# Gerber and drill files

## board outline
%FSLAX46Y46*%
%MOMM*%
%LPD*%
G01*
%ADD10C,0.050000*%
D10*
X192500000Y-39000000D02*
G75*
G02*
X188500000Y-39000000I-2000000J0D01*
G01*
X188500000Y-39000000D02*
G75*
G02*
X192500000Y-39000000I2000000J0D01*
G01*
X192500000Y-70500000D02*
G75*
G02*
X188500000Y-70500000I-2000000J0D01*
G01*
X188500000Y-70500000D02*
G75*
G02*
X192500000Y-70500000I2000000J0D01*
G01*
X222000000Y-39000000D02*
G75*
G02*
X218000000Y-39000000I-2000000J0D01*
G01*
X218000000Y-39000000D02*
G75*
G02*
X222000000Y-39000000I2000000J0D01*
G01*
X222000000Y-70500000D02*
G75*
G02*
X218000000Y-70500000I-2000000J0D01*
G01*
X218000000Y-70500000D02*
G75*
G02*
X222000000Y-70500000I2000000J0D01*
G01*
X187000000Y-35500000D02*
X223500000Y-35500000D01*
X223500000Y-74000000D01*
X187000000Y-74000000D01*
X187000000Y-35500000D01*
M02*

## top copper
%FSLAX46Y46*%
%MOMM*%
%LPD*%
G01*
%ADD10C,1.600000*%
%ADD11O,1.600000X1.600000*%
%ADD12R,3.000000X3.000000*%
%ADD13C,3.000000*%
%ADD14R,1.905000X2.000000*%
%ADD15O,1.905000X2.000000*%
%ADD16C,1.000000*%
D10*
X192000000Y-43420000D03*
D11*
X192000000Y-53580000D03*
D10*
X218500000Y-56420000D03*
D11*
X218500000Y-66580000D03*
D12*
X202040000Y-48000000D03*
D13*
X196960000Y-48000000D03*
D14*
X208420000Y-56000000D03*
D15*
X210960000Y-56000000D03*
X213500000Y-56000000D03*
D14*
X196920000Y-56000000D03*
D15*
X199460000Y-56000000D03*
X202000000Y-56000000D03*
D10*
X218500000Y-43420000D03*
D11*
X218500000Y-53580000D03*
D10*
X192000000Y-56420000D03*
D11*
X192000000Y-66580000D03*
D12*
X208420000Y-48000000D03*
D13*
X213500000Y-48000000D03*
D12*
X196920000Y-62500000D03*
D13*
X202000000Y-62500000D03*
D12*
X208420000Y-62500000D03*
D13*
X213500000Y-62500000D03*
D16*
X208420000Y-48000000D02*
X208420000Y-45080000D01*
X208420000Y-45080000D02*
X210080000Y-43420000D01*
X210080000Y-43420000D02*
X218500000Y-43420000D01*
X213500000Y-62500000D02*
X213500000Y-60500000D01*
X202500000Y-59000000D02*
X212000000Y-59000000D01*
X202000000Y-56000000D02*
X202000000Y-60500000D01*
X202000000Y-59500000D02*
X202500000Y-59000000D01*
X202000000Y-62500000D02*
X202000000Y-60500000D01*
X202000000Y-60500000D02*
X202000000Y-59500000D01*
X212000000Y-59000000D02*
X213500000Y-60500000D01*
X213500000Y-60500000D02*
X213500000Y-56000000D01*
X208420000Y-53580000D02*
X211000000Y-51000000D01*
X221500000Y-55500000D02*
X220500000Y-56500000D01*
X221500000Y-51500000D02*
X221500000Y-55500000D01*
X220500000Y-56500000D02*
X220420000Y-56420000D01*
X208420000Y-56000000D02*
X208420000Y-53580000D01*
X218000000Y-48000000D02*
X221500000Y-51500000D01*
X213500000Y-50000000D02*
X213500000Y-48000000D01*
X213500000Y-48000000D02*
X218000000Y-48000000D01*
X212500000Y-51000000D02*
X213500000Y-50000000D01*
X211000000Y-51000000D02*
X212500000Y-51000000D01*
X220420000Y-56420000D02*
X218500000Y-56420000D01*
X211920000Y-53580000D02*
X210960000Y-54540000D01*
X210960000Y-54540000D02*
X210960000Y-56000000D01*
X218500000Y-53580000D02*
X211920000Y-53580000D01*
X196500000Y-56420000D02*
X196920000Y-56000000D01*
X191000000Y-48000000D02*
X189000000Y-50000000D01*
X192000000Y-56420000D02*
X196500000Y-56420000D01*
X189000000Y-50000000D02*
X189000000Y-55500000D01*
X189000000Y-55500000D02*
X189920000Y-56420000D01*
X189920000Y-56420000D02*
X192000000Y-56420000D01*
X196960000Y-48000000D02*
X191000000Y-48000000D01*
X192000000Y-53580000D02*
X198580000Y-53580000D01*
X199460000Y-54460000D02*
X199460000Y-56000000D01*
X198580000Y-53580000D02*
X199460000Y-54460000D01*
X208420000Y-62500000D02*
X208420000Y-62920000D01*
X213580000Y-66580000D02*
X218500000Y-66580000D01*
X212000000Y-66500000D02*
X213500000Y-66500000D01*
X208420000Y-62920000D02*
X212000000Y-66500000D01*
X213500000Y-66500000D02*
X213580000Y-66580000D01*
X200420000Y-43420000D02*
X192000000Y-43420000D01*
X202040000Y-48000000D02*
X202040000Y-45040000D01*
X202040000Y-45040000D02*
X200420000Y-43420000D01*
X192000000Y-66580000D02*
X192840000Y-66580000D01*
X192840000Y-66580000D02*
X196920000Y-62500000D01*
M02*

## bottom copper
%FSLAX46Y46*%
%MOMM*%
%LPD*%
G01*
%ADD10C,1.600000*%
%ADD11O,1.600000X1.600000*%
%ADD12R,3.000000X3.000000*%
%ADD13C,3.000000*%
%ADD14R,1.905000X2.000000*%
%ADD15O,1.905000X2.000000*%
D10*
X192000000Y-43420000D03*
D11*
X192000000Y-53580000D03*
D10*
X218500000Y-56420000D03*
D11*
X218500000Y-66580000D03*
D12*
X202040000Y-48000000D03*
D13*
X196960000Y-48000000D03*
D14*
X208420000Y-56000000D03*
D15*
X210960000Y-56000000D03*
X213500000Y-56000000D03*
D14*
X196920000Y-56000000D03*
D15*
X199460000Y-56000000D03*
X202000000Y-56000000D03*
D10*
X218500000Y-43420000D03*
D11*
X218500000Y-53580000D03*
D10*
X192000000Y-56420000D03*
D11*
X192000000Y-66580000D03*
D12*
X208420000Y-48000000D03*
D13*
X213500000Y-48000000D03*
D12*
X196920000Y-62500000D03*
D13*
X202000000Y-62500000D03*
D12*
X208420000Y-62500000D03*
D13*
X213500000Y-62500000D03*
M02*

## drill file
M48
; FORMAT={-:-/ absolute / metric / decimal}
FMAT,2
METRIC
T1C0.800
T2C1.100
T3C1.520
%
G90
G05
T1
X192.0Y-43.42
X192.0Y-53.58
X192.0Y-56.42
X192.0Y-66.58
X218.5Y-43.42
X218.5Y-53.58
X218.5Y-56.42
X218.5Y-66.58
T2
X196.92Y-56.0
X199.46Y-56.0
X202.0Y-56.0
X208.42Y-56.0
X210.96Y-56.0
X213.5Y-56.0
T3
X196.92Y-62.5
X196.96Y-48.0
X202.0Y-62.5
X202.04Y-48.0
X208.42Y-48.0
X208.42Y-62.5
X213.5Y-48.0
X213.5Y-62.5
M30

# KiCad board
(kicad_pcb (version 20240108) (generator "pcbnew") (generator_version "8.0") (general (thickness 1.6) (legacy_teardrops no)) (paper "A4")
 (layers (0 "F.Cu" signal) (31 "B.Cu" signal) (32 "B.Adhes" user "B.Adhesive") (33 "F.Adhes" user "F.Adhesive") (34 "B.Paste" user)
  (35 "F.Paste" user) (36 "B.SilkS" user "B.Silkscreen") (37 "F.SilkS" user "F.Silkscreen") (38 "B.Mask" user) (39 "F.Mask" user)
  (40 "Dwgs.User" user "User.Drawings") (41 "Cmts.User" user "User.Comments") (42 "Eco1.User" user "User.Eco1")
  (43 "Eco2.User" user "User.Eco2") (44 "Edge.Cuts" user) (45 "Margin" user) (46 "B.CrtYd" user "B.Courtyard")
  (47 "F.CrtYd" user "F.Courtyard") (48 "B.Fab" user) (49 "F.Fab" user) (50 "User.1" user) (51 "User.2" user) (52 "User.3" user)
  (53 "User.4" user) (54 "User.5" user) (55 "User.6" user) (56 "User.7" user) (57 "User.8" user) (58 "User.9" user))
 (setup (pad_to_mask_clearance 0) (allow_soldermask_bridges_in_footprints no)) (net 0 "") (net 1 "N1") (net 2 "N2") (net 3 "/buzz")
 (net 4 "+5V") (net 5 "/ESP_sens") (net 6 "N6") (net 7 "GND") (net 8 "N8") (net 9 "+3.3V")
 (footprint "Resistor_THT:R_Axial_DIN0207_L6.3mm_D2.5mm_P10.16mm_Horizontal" (layer "F.Cu") (at 192 43.42 -90)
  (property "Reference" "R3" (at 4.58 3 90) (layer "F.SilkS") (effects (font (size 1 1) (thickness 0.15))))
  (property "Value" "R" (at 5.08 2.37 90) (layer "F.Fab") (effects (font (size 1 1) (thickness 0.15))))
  (pad "1" thru_hole circle (at 0 0 270) (size 1.6 1.6) (drill 0.8) (layers "*.Cu" "*.Mask") (remove_unused_layers no) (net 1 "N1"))
  (pad "2" thru_hole oval (at 10.16 0 270) (size 1.6 1.6) (drill 0.8) (layers "*.Cu" "*.Mask") (remove_unused_layers no) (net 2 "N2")))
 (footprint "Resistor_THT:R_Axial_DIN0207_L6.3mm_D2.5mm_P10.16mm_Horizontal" (layer "F.Cu") (at 218.5 56.42 -90)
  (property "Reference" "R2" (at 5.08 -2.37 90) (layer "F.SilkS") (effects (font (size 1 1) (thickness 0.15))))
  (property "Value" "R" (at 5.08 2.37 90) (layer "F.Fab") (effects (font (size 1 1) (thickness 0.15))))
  (pad "1" thru_hole circle (at 0 0 270) (size 1.6 1.6) (drill 0.8) (layers "*.Cu" "*.Mask") (remove_unused_layers no) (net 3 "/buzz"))
  (pad "2" thru_hole oval (at 10.16 0 270) (size 1.6 1.6) (drill 0.8) (layers "*.Cu" "*.Mask") (remove_unused_layers no) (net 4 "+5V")))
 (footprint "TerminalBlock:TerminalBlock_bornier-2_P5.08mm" (layer "F.Cu") (at 202.04 48 180)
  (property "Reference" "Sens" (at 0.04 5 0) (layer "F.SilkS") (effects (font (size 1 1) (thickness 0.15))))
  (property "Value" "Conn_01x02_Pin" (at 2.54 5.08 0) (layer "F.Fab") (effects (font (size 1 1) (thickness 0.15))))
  (pad "1" thru_hole rect (at 0 0 180) (size 3 3) (drill 1.52) (layers "*.Cu" "*.Mask") (remove_unused_layers no) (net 1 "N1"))
  (pad "2" thru_hole circle (at 5.08 0 180) (size 3 3) (drill 1.52) (layers "*.Cu" "*.Mask") (remove_unused_layers no) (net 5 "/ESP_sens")))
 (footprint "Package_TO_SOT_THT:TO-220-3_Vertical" (layer "F.Cu") (at 208.42 56)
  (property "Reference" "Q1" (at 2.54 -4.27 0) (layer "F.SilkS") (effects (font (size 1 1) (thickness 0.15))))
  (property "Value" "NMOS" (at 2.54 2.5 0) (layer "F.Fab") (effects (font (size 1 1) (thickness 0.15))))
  (pad "1" thru_hole rect (at 0 0) (size 1.905 2) (drill 1.1) (layers "*.Cu" "*.Mask") (remove_unused_layers no) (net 3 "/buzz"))
  (pad "2" thru_hole oval (at 2.54 0) (size 1.905 2) (drill 1.1) (layers "*.Cu" "*.Mask") (remove_unused_layers no) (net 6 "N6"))
  (pad "3" thru_hole oval (at 5.08 0) (size 1.905 2) (drill 1.1) (layers "*.Cu" "*.Mask") (remove_unused_layers no) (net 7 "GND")))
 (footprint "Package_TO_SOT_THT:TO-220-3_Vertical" (layer "F.Cu") (at 196.92 56)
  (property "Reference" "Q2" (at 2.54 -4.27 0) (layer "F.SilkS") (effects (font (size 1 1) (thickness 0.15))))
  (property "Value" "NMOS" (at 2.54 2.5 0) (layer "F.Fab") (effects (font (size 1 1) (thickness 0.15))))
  (pad "1" thru_hole rect (at 0 0) (size 1.905 2) (drill 1.1) (layers "*.Cu" "*.Mask") (remove_unused_layers no) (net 5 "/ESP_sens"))
  (pad "2" thru_hole oval (at 2.54 0) (size 1.905 2) (drill 1.1) (layers "*.Cu" "*.Mask") (remove_unused_layers no) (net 2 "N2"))
  (pad "3" thru_hole oval (at 5.08 0) (size 1.905 2) (drill 1.1) (layers "*.Cu" "*.Mask") (remove_unused_layers no) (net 7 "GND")))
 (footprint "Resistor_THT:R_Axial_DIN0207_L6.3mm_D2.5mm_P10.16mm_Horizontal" (layer "F.Cu") (at 218.5 43.42 -90)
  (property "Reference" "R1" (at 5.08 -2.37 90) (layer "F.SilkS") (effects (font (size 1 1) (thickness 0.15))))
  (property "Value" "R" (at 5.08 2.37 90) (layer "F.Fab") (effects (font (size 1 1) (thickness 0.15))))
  (pad "1" thru_hole circle (at 0 0 270) (size 1.6 1.6) (drill 0.8) (layers "*.Cu" "*.Mask") (remove_unused_layers no) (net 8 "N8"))
  (pad "2" thru_hole oval (at 10.16 0 270) (size 1.6 1.6) (drill 0.8) (layers "*.Cu" "*.Mask") (remove_unused_layers no) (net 6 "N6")))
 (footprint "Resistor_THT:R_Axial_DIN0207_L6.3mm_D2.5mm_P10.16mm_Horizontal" (layer "F.Cu") (at 192 56.42 -90)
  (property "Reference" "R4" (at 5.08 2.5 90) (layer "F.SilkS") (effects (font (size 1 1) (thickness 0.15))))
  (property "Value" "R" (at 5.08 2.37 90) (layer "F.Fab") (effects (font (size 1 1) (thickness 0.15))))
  (pad "1" thru_hole circle (at 0 0 270) (size 1.6 1.6) (drill 0.8) (layers "*.Cu" "*.Mask") (remove_unused_layers no) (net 5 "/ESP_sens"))
  (pad "2" thru_hole oval (at 10.16 0 270) (size 1.6 1.6) (drill 0.8) (layers "*.Cu" "*.Mask") (remove_unused_layers no) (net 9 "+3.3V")))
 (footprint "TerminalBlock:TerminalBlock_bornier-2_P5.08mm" (layer "F.Cu") (at 208.42 48)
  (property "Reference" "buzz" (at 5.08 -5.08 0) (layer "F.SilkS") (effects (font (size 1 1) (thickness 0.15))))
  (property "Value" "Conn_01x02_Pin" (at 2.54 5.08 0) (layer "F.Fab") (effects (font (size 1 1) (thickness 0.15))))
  (pad "1" thru_hole rect (at 0 0) (size 3 3) (drill 1.52) (layers "*.Cu" "*.Mask") (remove_unused_layers no) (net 8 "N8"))
  (pad "2" thru_hole circle (at 5.08 0) (size 3 3) (drill 1.52) (layers "*.Cu" "*.Mask") (remove_unused_layers no) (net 3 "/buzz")))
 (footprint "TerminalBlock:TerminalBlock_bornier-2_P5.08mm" (layer "F.Cu") (at 196.92 62.5)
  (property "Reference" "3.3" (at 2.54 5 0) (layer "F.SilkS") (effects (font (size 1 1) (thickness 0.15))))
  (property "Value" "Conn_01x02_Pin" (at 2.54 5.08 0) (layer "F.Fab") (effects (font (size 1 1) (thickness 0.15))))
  (pad "1" thru_hole rect (at 0 0) (size 3 3) (drill 1.52) (layers "*.Cu" "*.Mask") (remove_unused_layers no) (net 9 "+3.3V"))
  (pad "2" thru_hole circle (at 5.08 0) (size 3 3) (drill 1.52) (layers "*.Cu" "*.Mask") (remove_unused_layers no) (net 7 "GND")))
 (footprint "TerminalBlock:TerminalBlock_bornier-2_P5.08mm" (layer "F.Cu") (at 208.42 62.5)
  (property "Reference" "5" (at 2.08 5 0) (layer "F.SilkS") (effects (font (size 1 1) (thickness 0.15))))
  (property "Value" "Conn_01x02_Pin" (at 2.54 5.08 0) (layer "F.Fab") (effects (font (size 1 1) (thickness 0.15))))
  (pad "1" thru_hole rect (at 0 0) (size 3 3) (drill 1.52) (layers "*.Cu" "*.Mask") (remove_unused_layers no) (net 4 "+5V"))
  (pad "2" thru_hole circle (at 5.08 0) (size 3 3) (drill 1.52) (layers "*.Cu" "*.Mask") (remove_unused_layers no) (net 7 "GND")))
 (gr_circle (center 190.5 39) (end 192.5 39) (stroke (width 0.05) (type default)) (fill none) (layer "Edge.Cuts"))
 (gr_circle (center 190.5 70.5) (end 192.5 70.5) (stroke (width 0.05) (type default)) (fill none) (layer "Edge.Cuts"))
 (gr_circle (center 220 39) (end 222 39) (stroke (width 0.05) (type default)) (fill none) (layer "Edge.Cuts"))
 (gr_circle (center 220 70.5) (end 222 70.5) (stroke (width 0.05) (type default)) (fill none) (layer "Edge.Cuts"))
 (gr_rect (start 187 35.5) (end 223.5 74) (stroke (width 0.05) (type default)) (fill none) (layer "Edge.Cuts"))
 (segment (start 208.42 48) (end 208.42 45.08) (width 1) (layer "F.Cu") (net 8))
 (segment (start 208.42 45.08) (end 210.08 43.42) (width 1) (layer "F.Cu") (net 8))
 (segment (start 210.08 43.42) (end 218.5 43.42) (width 1) (layer "F.Cu") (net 8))
 (segment (start 213.5 62.5) (end 213.5 60.5) (width 1) (layer "F.Cu") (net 7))
 (segment (start 202.5 59) (end 212 59) (width 1) (layer "F.Cu") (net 7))
 (segment (start 202 56) (end 202 60.5) (width 1) (layer "F.Cu") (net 7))
 (segment (start 202 59.5) (end 202.5 59) (width 1) (layer "F.Cu") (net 7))
 (segment (start 202 62.5) (end 202 60.5) (width 1) (layer "F.Cu") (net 7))
 (segment (start 202 60.5) (end 202 59.5) (width 1) (layer "F.Cu") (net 7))
 (segment (start 212 59) (end 213.5 60.5) (width 1) (layer "F.Cu") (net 7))
 (segment (start 213.5 60.5) (end 213.5 56) (width 1) (layer "F.Cu") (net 7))
 (segment (start 208.42 53.58) (end 211 51) (width 1) (layer "F.Cu") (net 3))
 (segment (start 221.5 55.5) (end 220.5 56.5) (width 1) (layer "F.Cu") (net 3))
 (segment (start 221.5 51.5) (end 221.5 55.5) (width 1) (layer "F.Cu") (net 3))
 (segment (start 220.5 56.5) (end 220.42 56.42) (width 1) (layer "F.Cu") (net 3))
 (segment (start 208.42 56) (end 208.42 53.58) (width 1) (layer "F.Cu") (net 3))
 (segment (start 218 48) (end 221.5 51.5) (width 1) (layer "F.Cu") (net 3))
 (segment (start 213.5 50) (end 213.5 48) (width 1) (layer "F.Cu") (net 3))
 (segment (start 213.5 48) (end 218 48) (width 1) (layer "F.Cu") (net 3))
 (segment (start 212.5 51) (end 213.5 50) (width 1) (layer "F.Cu") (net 3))
 (segment (start 211 51) (end 212.5 51) (width 1) (layer "F.Cu") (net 3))
 (segment (start 220.42 56.42) (end 218.5 56.42) (width 1) (layer "F.Cu") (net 3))
 (segment (start 211.92 53.58) (end 210.96 54.54) (width 1) (layer "F.Cu") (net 6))
 (segment (start 210.96 54.54) (end 210.96 56) (width 1) (layer "F.Cu") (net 6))
 (segment (start 218.5 53.58) (end 211.92 53.58) (width 1) (layer "F.Cu") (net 6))
 (segment (start 196.5 56.42) (end 196.92 56) (width 1) (layer "F.Cu") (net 5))
 (segment (start 191 48) (end 189 50) (width 1) (layer "F.Cu") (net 5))
 (segment (start 192 56.42) (end 196.5 56.42) (width 1) (layer "F.Cu") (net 5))
 (segment (start 189 50) (end 189 55.5) (width 1) (layer "F.Cu") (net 5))
 (segment (start 189 55.5) (end 189.92 56.42) (width 1) (layer "F.Cu") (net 5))
 (segment (start 189.92 56.42) (end 192 56.42) (width 1) (layer "F.Cu") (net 5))
 (segment (start 196.96 48) (end 191 48) (width 1) (layer "F.Cu") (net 5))
 (segment (start 192 53.58) (end 198.58 53.58) (width 1) (layer "F.Cu") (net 2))
 (segment (start 199.46 54.46) (end 199.46 56) (width 1) (layer "F.Cu") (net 2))
 (segment (start 198.58 53.58) (end 199.46 54.46) (width 1) (layer "F.Cu") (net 2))
 (segment (start 208.42 62.5) (end 208.42 62.92) (width 1) (layer "F.Cu") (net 4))
 (segment (start 213.58 66.58) (end 218.5 66.58) (width 1) (layer "F.Cu") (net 4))
 (segment (start 212 66.5) (end 213.5 66.5) (width 1) (layer "F.Cu") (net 4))
 (segment (start 208.42 62.92) (end 212 66.5) (width 1) (layer "F.Cu") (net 4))
 (segment (start 213.5 66.5) (end 213.58 66.58) (width 1) (layer "F.Cu") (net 4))
 (segment (start 200.42 43.42) (end 192 43.42) (width 1) (layer "F.Cu") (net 1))
 (segment (start 202.04 48) (end 202.04 45.04) (width 1) (layer "F.Cu") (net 1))
 (segment (start 202.04 45.04) (end 200.42 43.42) (width 1) (layer "F.Cu") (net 1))
 (segment (start 192 66.58) (end 192.84 66.58) (width 1) (layer "F.Cu") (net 9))
 (segment (start 192.84 66.58) (end 196.92 62.5) (width 1) (layer "F.Cu") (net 9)))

